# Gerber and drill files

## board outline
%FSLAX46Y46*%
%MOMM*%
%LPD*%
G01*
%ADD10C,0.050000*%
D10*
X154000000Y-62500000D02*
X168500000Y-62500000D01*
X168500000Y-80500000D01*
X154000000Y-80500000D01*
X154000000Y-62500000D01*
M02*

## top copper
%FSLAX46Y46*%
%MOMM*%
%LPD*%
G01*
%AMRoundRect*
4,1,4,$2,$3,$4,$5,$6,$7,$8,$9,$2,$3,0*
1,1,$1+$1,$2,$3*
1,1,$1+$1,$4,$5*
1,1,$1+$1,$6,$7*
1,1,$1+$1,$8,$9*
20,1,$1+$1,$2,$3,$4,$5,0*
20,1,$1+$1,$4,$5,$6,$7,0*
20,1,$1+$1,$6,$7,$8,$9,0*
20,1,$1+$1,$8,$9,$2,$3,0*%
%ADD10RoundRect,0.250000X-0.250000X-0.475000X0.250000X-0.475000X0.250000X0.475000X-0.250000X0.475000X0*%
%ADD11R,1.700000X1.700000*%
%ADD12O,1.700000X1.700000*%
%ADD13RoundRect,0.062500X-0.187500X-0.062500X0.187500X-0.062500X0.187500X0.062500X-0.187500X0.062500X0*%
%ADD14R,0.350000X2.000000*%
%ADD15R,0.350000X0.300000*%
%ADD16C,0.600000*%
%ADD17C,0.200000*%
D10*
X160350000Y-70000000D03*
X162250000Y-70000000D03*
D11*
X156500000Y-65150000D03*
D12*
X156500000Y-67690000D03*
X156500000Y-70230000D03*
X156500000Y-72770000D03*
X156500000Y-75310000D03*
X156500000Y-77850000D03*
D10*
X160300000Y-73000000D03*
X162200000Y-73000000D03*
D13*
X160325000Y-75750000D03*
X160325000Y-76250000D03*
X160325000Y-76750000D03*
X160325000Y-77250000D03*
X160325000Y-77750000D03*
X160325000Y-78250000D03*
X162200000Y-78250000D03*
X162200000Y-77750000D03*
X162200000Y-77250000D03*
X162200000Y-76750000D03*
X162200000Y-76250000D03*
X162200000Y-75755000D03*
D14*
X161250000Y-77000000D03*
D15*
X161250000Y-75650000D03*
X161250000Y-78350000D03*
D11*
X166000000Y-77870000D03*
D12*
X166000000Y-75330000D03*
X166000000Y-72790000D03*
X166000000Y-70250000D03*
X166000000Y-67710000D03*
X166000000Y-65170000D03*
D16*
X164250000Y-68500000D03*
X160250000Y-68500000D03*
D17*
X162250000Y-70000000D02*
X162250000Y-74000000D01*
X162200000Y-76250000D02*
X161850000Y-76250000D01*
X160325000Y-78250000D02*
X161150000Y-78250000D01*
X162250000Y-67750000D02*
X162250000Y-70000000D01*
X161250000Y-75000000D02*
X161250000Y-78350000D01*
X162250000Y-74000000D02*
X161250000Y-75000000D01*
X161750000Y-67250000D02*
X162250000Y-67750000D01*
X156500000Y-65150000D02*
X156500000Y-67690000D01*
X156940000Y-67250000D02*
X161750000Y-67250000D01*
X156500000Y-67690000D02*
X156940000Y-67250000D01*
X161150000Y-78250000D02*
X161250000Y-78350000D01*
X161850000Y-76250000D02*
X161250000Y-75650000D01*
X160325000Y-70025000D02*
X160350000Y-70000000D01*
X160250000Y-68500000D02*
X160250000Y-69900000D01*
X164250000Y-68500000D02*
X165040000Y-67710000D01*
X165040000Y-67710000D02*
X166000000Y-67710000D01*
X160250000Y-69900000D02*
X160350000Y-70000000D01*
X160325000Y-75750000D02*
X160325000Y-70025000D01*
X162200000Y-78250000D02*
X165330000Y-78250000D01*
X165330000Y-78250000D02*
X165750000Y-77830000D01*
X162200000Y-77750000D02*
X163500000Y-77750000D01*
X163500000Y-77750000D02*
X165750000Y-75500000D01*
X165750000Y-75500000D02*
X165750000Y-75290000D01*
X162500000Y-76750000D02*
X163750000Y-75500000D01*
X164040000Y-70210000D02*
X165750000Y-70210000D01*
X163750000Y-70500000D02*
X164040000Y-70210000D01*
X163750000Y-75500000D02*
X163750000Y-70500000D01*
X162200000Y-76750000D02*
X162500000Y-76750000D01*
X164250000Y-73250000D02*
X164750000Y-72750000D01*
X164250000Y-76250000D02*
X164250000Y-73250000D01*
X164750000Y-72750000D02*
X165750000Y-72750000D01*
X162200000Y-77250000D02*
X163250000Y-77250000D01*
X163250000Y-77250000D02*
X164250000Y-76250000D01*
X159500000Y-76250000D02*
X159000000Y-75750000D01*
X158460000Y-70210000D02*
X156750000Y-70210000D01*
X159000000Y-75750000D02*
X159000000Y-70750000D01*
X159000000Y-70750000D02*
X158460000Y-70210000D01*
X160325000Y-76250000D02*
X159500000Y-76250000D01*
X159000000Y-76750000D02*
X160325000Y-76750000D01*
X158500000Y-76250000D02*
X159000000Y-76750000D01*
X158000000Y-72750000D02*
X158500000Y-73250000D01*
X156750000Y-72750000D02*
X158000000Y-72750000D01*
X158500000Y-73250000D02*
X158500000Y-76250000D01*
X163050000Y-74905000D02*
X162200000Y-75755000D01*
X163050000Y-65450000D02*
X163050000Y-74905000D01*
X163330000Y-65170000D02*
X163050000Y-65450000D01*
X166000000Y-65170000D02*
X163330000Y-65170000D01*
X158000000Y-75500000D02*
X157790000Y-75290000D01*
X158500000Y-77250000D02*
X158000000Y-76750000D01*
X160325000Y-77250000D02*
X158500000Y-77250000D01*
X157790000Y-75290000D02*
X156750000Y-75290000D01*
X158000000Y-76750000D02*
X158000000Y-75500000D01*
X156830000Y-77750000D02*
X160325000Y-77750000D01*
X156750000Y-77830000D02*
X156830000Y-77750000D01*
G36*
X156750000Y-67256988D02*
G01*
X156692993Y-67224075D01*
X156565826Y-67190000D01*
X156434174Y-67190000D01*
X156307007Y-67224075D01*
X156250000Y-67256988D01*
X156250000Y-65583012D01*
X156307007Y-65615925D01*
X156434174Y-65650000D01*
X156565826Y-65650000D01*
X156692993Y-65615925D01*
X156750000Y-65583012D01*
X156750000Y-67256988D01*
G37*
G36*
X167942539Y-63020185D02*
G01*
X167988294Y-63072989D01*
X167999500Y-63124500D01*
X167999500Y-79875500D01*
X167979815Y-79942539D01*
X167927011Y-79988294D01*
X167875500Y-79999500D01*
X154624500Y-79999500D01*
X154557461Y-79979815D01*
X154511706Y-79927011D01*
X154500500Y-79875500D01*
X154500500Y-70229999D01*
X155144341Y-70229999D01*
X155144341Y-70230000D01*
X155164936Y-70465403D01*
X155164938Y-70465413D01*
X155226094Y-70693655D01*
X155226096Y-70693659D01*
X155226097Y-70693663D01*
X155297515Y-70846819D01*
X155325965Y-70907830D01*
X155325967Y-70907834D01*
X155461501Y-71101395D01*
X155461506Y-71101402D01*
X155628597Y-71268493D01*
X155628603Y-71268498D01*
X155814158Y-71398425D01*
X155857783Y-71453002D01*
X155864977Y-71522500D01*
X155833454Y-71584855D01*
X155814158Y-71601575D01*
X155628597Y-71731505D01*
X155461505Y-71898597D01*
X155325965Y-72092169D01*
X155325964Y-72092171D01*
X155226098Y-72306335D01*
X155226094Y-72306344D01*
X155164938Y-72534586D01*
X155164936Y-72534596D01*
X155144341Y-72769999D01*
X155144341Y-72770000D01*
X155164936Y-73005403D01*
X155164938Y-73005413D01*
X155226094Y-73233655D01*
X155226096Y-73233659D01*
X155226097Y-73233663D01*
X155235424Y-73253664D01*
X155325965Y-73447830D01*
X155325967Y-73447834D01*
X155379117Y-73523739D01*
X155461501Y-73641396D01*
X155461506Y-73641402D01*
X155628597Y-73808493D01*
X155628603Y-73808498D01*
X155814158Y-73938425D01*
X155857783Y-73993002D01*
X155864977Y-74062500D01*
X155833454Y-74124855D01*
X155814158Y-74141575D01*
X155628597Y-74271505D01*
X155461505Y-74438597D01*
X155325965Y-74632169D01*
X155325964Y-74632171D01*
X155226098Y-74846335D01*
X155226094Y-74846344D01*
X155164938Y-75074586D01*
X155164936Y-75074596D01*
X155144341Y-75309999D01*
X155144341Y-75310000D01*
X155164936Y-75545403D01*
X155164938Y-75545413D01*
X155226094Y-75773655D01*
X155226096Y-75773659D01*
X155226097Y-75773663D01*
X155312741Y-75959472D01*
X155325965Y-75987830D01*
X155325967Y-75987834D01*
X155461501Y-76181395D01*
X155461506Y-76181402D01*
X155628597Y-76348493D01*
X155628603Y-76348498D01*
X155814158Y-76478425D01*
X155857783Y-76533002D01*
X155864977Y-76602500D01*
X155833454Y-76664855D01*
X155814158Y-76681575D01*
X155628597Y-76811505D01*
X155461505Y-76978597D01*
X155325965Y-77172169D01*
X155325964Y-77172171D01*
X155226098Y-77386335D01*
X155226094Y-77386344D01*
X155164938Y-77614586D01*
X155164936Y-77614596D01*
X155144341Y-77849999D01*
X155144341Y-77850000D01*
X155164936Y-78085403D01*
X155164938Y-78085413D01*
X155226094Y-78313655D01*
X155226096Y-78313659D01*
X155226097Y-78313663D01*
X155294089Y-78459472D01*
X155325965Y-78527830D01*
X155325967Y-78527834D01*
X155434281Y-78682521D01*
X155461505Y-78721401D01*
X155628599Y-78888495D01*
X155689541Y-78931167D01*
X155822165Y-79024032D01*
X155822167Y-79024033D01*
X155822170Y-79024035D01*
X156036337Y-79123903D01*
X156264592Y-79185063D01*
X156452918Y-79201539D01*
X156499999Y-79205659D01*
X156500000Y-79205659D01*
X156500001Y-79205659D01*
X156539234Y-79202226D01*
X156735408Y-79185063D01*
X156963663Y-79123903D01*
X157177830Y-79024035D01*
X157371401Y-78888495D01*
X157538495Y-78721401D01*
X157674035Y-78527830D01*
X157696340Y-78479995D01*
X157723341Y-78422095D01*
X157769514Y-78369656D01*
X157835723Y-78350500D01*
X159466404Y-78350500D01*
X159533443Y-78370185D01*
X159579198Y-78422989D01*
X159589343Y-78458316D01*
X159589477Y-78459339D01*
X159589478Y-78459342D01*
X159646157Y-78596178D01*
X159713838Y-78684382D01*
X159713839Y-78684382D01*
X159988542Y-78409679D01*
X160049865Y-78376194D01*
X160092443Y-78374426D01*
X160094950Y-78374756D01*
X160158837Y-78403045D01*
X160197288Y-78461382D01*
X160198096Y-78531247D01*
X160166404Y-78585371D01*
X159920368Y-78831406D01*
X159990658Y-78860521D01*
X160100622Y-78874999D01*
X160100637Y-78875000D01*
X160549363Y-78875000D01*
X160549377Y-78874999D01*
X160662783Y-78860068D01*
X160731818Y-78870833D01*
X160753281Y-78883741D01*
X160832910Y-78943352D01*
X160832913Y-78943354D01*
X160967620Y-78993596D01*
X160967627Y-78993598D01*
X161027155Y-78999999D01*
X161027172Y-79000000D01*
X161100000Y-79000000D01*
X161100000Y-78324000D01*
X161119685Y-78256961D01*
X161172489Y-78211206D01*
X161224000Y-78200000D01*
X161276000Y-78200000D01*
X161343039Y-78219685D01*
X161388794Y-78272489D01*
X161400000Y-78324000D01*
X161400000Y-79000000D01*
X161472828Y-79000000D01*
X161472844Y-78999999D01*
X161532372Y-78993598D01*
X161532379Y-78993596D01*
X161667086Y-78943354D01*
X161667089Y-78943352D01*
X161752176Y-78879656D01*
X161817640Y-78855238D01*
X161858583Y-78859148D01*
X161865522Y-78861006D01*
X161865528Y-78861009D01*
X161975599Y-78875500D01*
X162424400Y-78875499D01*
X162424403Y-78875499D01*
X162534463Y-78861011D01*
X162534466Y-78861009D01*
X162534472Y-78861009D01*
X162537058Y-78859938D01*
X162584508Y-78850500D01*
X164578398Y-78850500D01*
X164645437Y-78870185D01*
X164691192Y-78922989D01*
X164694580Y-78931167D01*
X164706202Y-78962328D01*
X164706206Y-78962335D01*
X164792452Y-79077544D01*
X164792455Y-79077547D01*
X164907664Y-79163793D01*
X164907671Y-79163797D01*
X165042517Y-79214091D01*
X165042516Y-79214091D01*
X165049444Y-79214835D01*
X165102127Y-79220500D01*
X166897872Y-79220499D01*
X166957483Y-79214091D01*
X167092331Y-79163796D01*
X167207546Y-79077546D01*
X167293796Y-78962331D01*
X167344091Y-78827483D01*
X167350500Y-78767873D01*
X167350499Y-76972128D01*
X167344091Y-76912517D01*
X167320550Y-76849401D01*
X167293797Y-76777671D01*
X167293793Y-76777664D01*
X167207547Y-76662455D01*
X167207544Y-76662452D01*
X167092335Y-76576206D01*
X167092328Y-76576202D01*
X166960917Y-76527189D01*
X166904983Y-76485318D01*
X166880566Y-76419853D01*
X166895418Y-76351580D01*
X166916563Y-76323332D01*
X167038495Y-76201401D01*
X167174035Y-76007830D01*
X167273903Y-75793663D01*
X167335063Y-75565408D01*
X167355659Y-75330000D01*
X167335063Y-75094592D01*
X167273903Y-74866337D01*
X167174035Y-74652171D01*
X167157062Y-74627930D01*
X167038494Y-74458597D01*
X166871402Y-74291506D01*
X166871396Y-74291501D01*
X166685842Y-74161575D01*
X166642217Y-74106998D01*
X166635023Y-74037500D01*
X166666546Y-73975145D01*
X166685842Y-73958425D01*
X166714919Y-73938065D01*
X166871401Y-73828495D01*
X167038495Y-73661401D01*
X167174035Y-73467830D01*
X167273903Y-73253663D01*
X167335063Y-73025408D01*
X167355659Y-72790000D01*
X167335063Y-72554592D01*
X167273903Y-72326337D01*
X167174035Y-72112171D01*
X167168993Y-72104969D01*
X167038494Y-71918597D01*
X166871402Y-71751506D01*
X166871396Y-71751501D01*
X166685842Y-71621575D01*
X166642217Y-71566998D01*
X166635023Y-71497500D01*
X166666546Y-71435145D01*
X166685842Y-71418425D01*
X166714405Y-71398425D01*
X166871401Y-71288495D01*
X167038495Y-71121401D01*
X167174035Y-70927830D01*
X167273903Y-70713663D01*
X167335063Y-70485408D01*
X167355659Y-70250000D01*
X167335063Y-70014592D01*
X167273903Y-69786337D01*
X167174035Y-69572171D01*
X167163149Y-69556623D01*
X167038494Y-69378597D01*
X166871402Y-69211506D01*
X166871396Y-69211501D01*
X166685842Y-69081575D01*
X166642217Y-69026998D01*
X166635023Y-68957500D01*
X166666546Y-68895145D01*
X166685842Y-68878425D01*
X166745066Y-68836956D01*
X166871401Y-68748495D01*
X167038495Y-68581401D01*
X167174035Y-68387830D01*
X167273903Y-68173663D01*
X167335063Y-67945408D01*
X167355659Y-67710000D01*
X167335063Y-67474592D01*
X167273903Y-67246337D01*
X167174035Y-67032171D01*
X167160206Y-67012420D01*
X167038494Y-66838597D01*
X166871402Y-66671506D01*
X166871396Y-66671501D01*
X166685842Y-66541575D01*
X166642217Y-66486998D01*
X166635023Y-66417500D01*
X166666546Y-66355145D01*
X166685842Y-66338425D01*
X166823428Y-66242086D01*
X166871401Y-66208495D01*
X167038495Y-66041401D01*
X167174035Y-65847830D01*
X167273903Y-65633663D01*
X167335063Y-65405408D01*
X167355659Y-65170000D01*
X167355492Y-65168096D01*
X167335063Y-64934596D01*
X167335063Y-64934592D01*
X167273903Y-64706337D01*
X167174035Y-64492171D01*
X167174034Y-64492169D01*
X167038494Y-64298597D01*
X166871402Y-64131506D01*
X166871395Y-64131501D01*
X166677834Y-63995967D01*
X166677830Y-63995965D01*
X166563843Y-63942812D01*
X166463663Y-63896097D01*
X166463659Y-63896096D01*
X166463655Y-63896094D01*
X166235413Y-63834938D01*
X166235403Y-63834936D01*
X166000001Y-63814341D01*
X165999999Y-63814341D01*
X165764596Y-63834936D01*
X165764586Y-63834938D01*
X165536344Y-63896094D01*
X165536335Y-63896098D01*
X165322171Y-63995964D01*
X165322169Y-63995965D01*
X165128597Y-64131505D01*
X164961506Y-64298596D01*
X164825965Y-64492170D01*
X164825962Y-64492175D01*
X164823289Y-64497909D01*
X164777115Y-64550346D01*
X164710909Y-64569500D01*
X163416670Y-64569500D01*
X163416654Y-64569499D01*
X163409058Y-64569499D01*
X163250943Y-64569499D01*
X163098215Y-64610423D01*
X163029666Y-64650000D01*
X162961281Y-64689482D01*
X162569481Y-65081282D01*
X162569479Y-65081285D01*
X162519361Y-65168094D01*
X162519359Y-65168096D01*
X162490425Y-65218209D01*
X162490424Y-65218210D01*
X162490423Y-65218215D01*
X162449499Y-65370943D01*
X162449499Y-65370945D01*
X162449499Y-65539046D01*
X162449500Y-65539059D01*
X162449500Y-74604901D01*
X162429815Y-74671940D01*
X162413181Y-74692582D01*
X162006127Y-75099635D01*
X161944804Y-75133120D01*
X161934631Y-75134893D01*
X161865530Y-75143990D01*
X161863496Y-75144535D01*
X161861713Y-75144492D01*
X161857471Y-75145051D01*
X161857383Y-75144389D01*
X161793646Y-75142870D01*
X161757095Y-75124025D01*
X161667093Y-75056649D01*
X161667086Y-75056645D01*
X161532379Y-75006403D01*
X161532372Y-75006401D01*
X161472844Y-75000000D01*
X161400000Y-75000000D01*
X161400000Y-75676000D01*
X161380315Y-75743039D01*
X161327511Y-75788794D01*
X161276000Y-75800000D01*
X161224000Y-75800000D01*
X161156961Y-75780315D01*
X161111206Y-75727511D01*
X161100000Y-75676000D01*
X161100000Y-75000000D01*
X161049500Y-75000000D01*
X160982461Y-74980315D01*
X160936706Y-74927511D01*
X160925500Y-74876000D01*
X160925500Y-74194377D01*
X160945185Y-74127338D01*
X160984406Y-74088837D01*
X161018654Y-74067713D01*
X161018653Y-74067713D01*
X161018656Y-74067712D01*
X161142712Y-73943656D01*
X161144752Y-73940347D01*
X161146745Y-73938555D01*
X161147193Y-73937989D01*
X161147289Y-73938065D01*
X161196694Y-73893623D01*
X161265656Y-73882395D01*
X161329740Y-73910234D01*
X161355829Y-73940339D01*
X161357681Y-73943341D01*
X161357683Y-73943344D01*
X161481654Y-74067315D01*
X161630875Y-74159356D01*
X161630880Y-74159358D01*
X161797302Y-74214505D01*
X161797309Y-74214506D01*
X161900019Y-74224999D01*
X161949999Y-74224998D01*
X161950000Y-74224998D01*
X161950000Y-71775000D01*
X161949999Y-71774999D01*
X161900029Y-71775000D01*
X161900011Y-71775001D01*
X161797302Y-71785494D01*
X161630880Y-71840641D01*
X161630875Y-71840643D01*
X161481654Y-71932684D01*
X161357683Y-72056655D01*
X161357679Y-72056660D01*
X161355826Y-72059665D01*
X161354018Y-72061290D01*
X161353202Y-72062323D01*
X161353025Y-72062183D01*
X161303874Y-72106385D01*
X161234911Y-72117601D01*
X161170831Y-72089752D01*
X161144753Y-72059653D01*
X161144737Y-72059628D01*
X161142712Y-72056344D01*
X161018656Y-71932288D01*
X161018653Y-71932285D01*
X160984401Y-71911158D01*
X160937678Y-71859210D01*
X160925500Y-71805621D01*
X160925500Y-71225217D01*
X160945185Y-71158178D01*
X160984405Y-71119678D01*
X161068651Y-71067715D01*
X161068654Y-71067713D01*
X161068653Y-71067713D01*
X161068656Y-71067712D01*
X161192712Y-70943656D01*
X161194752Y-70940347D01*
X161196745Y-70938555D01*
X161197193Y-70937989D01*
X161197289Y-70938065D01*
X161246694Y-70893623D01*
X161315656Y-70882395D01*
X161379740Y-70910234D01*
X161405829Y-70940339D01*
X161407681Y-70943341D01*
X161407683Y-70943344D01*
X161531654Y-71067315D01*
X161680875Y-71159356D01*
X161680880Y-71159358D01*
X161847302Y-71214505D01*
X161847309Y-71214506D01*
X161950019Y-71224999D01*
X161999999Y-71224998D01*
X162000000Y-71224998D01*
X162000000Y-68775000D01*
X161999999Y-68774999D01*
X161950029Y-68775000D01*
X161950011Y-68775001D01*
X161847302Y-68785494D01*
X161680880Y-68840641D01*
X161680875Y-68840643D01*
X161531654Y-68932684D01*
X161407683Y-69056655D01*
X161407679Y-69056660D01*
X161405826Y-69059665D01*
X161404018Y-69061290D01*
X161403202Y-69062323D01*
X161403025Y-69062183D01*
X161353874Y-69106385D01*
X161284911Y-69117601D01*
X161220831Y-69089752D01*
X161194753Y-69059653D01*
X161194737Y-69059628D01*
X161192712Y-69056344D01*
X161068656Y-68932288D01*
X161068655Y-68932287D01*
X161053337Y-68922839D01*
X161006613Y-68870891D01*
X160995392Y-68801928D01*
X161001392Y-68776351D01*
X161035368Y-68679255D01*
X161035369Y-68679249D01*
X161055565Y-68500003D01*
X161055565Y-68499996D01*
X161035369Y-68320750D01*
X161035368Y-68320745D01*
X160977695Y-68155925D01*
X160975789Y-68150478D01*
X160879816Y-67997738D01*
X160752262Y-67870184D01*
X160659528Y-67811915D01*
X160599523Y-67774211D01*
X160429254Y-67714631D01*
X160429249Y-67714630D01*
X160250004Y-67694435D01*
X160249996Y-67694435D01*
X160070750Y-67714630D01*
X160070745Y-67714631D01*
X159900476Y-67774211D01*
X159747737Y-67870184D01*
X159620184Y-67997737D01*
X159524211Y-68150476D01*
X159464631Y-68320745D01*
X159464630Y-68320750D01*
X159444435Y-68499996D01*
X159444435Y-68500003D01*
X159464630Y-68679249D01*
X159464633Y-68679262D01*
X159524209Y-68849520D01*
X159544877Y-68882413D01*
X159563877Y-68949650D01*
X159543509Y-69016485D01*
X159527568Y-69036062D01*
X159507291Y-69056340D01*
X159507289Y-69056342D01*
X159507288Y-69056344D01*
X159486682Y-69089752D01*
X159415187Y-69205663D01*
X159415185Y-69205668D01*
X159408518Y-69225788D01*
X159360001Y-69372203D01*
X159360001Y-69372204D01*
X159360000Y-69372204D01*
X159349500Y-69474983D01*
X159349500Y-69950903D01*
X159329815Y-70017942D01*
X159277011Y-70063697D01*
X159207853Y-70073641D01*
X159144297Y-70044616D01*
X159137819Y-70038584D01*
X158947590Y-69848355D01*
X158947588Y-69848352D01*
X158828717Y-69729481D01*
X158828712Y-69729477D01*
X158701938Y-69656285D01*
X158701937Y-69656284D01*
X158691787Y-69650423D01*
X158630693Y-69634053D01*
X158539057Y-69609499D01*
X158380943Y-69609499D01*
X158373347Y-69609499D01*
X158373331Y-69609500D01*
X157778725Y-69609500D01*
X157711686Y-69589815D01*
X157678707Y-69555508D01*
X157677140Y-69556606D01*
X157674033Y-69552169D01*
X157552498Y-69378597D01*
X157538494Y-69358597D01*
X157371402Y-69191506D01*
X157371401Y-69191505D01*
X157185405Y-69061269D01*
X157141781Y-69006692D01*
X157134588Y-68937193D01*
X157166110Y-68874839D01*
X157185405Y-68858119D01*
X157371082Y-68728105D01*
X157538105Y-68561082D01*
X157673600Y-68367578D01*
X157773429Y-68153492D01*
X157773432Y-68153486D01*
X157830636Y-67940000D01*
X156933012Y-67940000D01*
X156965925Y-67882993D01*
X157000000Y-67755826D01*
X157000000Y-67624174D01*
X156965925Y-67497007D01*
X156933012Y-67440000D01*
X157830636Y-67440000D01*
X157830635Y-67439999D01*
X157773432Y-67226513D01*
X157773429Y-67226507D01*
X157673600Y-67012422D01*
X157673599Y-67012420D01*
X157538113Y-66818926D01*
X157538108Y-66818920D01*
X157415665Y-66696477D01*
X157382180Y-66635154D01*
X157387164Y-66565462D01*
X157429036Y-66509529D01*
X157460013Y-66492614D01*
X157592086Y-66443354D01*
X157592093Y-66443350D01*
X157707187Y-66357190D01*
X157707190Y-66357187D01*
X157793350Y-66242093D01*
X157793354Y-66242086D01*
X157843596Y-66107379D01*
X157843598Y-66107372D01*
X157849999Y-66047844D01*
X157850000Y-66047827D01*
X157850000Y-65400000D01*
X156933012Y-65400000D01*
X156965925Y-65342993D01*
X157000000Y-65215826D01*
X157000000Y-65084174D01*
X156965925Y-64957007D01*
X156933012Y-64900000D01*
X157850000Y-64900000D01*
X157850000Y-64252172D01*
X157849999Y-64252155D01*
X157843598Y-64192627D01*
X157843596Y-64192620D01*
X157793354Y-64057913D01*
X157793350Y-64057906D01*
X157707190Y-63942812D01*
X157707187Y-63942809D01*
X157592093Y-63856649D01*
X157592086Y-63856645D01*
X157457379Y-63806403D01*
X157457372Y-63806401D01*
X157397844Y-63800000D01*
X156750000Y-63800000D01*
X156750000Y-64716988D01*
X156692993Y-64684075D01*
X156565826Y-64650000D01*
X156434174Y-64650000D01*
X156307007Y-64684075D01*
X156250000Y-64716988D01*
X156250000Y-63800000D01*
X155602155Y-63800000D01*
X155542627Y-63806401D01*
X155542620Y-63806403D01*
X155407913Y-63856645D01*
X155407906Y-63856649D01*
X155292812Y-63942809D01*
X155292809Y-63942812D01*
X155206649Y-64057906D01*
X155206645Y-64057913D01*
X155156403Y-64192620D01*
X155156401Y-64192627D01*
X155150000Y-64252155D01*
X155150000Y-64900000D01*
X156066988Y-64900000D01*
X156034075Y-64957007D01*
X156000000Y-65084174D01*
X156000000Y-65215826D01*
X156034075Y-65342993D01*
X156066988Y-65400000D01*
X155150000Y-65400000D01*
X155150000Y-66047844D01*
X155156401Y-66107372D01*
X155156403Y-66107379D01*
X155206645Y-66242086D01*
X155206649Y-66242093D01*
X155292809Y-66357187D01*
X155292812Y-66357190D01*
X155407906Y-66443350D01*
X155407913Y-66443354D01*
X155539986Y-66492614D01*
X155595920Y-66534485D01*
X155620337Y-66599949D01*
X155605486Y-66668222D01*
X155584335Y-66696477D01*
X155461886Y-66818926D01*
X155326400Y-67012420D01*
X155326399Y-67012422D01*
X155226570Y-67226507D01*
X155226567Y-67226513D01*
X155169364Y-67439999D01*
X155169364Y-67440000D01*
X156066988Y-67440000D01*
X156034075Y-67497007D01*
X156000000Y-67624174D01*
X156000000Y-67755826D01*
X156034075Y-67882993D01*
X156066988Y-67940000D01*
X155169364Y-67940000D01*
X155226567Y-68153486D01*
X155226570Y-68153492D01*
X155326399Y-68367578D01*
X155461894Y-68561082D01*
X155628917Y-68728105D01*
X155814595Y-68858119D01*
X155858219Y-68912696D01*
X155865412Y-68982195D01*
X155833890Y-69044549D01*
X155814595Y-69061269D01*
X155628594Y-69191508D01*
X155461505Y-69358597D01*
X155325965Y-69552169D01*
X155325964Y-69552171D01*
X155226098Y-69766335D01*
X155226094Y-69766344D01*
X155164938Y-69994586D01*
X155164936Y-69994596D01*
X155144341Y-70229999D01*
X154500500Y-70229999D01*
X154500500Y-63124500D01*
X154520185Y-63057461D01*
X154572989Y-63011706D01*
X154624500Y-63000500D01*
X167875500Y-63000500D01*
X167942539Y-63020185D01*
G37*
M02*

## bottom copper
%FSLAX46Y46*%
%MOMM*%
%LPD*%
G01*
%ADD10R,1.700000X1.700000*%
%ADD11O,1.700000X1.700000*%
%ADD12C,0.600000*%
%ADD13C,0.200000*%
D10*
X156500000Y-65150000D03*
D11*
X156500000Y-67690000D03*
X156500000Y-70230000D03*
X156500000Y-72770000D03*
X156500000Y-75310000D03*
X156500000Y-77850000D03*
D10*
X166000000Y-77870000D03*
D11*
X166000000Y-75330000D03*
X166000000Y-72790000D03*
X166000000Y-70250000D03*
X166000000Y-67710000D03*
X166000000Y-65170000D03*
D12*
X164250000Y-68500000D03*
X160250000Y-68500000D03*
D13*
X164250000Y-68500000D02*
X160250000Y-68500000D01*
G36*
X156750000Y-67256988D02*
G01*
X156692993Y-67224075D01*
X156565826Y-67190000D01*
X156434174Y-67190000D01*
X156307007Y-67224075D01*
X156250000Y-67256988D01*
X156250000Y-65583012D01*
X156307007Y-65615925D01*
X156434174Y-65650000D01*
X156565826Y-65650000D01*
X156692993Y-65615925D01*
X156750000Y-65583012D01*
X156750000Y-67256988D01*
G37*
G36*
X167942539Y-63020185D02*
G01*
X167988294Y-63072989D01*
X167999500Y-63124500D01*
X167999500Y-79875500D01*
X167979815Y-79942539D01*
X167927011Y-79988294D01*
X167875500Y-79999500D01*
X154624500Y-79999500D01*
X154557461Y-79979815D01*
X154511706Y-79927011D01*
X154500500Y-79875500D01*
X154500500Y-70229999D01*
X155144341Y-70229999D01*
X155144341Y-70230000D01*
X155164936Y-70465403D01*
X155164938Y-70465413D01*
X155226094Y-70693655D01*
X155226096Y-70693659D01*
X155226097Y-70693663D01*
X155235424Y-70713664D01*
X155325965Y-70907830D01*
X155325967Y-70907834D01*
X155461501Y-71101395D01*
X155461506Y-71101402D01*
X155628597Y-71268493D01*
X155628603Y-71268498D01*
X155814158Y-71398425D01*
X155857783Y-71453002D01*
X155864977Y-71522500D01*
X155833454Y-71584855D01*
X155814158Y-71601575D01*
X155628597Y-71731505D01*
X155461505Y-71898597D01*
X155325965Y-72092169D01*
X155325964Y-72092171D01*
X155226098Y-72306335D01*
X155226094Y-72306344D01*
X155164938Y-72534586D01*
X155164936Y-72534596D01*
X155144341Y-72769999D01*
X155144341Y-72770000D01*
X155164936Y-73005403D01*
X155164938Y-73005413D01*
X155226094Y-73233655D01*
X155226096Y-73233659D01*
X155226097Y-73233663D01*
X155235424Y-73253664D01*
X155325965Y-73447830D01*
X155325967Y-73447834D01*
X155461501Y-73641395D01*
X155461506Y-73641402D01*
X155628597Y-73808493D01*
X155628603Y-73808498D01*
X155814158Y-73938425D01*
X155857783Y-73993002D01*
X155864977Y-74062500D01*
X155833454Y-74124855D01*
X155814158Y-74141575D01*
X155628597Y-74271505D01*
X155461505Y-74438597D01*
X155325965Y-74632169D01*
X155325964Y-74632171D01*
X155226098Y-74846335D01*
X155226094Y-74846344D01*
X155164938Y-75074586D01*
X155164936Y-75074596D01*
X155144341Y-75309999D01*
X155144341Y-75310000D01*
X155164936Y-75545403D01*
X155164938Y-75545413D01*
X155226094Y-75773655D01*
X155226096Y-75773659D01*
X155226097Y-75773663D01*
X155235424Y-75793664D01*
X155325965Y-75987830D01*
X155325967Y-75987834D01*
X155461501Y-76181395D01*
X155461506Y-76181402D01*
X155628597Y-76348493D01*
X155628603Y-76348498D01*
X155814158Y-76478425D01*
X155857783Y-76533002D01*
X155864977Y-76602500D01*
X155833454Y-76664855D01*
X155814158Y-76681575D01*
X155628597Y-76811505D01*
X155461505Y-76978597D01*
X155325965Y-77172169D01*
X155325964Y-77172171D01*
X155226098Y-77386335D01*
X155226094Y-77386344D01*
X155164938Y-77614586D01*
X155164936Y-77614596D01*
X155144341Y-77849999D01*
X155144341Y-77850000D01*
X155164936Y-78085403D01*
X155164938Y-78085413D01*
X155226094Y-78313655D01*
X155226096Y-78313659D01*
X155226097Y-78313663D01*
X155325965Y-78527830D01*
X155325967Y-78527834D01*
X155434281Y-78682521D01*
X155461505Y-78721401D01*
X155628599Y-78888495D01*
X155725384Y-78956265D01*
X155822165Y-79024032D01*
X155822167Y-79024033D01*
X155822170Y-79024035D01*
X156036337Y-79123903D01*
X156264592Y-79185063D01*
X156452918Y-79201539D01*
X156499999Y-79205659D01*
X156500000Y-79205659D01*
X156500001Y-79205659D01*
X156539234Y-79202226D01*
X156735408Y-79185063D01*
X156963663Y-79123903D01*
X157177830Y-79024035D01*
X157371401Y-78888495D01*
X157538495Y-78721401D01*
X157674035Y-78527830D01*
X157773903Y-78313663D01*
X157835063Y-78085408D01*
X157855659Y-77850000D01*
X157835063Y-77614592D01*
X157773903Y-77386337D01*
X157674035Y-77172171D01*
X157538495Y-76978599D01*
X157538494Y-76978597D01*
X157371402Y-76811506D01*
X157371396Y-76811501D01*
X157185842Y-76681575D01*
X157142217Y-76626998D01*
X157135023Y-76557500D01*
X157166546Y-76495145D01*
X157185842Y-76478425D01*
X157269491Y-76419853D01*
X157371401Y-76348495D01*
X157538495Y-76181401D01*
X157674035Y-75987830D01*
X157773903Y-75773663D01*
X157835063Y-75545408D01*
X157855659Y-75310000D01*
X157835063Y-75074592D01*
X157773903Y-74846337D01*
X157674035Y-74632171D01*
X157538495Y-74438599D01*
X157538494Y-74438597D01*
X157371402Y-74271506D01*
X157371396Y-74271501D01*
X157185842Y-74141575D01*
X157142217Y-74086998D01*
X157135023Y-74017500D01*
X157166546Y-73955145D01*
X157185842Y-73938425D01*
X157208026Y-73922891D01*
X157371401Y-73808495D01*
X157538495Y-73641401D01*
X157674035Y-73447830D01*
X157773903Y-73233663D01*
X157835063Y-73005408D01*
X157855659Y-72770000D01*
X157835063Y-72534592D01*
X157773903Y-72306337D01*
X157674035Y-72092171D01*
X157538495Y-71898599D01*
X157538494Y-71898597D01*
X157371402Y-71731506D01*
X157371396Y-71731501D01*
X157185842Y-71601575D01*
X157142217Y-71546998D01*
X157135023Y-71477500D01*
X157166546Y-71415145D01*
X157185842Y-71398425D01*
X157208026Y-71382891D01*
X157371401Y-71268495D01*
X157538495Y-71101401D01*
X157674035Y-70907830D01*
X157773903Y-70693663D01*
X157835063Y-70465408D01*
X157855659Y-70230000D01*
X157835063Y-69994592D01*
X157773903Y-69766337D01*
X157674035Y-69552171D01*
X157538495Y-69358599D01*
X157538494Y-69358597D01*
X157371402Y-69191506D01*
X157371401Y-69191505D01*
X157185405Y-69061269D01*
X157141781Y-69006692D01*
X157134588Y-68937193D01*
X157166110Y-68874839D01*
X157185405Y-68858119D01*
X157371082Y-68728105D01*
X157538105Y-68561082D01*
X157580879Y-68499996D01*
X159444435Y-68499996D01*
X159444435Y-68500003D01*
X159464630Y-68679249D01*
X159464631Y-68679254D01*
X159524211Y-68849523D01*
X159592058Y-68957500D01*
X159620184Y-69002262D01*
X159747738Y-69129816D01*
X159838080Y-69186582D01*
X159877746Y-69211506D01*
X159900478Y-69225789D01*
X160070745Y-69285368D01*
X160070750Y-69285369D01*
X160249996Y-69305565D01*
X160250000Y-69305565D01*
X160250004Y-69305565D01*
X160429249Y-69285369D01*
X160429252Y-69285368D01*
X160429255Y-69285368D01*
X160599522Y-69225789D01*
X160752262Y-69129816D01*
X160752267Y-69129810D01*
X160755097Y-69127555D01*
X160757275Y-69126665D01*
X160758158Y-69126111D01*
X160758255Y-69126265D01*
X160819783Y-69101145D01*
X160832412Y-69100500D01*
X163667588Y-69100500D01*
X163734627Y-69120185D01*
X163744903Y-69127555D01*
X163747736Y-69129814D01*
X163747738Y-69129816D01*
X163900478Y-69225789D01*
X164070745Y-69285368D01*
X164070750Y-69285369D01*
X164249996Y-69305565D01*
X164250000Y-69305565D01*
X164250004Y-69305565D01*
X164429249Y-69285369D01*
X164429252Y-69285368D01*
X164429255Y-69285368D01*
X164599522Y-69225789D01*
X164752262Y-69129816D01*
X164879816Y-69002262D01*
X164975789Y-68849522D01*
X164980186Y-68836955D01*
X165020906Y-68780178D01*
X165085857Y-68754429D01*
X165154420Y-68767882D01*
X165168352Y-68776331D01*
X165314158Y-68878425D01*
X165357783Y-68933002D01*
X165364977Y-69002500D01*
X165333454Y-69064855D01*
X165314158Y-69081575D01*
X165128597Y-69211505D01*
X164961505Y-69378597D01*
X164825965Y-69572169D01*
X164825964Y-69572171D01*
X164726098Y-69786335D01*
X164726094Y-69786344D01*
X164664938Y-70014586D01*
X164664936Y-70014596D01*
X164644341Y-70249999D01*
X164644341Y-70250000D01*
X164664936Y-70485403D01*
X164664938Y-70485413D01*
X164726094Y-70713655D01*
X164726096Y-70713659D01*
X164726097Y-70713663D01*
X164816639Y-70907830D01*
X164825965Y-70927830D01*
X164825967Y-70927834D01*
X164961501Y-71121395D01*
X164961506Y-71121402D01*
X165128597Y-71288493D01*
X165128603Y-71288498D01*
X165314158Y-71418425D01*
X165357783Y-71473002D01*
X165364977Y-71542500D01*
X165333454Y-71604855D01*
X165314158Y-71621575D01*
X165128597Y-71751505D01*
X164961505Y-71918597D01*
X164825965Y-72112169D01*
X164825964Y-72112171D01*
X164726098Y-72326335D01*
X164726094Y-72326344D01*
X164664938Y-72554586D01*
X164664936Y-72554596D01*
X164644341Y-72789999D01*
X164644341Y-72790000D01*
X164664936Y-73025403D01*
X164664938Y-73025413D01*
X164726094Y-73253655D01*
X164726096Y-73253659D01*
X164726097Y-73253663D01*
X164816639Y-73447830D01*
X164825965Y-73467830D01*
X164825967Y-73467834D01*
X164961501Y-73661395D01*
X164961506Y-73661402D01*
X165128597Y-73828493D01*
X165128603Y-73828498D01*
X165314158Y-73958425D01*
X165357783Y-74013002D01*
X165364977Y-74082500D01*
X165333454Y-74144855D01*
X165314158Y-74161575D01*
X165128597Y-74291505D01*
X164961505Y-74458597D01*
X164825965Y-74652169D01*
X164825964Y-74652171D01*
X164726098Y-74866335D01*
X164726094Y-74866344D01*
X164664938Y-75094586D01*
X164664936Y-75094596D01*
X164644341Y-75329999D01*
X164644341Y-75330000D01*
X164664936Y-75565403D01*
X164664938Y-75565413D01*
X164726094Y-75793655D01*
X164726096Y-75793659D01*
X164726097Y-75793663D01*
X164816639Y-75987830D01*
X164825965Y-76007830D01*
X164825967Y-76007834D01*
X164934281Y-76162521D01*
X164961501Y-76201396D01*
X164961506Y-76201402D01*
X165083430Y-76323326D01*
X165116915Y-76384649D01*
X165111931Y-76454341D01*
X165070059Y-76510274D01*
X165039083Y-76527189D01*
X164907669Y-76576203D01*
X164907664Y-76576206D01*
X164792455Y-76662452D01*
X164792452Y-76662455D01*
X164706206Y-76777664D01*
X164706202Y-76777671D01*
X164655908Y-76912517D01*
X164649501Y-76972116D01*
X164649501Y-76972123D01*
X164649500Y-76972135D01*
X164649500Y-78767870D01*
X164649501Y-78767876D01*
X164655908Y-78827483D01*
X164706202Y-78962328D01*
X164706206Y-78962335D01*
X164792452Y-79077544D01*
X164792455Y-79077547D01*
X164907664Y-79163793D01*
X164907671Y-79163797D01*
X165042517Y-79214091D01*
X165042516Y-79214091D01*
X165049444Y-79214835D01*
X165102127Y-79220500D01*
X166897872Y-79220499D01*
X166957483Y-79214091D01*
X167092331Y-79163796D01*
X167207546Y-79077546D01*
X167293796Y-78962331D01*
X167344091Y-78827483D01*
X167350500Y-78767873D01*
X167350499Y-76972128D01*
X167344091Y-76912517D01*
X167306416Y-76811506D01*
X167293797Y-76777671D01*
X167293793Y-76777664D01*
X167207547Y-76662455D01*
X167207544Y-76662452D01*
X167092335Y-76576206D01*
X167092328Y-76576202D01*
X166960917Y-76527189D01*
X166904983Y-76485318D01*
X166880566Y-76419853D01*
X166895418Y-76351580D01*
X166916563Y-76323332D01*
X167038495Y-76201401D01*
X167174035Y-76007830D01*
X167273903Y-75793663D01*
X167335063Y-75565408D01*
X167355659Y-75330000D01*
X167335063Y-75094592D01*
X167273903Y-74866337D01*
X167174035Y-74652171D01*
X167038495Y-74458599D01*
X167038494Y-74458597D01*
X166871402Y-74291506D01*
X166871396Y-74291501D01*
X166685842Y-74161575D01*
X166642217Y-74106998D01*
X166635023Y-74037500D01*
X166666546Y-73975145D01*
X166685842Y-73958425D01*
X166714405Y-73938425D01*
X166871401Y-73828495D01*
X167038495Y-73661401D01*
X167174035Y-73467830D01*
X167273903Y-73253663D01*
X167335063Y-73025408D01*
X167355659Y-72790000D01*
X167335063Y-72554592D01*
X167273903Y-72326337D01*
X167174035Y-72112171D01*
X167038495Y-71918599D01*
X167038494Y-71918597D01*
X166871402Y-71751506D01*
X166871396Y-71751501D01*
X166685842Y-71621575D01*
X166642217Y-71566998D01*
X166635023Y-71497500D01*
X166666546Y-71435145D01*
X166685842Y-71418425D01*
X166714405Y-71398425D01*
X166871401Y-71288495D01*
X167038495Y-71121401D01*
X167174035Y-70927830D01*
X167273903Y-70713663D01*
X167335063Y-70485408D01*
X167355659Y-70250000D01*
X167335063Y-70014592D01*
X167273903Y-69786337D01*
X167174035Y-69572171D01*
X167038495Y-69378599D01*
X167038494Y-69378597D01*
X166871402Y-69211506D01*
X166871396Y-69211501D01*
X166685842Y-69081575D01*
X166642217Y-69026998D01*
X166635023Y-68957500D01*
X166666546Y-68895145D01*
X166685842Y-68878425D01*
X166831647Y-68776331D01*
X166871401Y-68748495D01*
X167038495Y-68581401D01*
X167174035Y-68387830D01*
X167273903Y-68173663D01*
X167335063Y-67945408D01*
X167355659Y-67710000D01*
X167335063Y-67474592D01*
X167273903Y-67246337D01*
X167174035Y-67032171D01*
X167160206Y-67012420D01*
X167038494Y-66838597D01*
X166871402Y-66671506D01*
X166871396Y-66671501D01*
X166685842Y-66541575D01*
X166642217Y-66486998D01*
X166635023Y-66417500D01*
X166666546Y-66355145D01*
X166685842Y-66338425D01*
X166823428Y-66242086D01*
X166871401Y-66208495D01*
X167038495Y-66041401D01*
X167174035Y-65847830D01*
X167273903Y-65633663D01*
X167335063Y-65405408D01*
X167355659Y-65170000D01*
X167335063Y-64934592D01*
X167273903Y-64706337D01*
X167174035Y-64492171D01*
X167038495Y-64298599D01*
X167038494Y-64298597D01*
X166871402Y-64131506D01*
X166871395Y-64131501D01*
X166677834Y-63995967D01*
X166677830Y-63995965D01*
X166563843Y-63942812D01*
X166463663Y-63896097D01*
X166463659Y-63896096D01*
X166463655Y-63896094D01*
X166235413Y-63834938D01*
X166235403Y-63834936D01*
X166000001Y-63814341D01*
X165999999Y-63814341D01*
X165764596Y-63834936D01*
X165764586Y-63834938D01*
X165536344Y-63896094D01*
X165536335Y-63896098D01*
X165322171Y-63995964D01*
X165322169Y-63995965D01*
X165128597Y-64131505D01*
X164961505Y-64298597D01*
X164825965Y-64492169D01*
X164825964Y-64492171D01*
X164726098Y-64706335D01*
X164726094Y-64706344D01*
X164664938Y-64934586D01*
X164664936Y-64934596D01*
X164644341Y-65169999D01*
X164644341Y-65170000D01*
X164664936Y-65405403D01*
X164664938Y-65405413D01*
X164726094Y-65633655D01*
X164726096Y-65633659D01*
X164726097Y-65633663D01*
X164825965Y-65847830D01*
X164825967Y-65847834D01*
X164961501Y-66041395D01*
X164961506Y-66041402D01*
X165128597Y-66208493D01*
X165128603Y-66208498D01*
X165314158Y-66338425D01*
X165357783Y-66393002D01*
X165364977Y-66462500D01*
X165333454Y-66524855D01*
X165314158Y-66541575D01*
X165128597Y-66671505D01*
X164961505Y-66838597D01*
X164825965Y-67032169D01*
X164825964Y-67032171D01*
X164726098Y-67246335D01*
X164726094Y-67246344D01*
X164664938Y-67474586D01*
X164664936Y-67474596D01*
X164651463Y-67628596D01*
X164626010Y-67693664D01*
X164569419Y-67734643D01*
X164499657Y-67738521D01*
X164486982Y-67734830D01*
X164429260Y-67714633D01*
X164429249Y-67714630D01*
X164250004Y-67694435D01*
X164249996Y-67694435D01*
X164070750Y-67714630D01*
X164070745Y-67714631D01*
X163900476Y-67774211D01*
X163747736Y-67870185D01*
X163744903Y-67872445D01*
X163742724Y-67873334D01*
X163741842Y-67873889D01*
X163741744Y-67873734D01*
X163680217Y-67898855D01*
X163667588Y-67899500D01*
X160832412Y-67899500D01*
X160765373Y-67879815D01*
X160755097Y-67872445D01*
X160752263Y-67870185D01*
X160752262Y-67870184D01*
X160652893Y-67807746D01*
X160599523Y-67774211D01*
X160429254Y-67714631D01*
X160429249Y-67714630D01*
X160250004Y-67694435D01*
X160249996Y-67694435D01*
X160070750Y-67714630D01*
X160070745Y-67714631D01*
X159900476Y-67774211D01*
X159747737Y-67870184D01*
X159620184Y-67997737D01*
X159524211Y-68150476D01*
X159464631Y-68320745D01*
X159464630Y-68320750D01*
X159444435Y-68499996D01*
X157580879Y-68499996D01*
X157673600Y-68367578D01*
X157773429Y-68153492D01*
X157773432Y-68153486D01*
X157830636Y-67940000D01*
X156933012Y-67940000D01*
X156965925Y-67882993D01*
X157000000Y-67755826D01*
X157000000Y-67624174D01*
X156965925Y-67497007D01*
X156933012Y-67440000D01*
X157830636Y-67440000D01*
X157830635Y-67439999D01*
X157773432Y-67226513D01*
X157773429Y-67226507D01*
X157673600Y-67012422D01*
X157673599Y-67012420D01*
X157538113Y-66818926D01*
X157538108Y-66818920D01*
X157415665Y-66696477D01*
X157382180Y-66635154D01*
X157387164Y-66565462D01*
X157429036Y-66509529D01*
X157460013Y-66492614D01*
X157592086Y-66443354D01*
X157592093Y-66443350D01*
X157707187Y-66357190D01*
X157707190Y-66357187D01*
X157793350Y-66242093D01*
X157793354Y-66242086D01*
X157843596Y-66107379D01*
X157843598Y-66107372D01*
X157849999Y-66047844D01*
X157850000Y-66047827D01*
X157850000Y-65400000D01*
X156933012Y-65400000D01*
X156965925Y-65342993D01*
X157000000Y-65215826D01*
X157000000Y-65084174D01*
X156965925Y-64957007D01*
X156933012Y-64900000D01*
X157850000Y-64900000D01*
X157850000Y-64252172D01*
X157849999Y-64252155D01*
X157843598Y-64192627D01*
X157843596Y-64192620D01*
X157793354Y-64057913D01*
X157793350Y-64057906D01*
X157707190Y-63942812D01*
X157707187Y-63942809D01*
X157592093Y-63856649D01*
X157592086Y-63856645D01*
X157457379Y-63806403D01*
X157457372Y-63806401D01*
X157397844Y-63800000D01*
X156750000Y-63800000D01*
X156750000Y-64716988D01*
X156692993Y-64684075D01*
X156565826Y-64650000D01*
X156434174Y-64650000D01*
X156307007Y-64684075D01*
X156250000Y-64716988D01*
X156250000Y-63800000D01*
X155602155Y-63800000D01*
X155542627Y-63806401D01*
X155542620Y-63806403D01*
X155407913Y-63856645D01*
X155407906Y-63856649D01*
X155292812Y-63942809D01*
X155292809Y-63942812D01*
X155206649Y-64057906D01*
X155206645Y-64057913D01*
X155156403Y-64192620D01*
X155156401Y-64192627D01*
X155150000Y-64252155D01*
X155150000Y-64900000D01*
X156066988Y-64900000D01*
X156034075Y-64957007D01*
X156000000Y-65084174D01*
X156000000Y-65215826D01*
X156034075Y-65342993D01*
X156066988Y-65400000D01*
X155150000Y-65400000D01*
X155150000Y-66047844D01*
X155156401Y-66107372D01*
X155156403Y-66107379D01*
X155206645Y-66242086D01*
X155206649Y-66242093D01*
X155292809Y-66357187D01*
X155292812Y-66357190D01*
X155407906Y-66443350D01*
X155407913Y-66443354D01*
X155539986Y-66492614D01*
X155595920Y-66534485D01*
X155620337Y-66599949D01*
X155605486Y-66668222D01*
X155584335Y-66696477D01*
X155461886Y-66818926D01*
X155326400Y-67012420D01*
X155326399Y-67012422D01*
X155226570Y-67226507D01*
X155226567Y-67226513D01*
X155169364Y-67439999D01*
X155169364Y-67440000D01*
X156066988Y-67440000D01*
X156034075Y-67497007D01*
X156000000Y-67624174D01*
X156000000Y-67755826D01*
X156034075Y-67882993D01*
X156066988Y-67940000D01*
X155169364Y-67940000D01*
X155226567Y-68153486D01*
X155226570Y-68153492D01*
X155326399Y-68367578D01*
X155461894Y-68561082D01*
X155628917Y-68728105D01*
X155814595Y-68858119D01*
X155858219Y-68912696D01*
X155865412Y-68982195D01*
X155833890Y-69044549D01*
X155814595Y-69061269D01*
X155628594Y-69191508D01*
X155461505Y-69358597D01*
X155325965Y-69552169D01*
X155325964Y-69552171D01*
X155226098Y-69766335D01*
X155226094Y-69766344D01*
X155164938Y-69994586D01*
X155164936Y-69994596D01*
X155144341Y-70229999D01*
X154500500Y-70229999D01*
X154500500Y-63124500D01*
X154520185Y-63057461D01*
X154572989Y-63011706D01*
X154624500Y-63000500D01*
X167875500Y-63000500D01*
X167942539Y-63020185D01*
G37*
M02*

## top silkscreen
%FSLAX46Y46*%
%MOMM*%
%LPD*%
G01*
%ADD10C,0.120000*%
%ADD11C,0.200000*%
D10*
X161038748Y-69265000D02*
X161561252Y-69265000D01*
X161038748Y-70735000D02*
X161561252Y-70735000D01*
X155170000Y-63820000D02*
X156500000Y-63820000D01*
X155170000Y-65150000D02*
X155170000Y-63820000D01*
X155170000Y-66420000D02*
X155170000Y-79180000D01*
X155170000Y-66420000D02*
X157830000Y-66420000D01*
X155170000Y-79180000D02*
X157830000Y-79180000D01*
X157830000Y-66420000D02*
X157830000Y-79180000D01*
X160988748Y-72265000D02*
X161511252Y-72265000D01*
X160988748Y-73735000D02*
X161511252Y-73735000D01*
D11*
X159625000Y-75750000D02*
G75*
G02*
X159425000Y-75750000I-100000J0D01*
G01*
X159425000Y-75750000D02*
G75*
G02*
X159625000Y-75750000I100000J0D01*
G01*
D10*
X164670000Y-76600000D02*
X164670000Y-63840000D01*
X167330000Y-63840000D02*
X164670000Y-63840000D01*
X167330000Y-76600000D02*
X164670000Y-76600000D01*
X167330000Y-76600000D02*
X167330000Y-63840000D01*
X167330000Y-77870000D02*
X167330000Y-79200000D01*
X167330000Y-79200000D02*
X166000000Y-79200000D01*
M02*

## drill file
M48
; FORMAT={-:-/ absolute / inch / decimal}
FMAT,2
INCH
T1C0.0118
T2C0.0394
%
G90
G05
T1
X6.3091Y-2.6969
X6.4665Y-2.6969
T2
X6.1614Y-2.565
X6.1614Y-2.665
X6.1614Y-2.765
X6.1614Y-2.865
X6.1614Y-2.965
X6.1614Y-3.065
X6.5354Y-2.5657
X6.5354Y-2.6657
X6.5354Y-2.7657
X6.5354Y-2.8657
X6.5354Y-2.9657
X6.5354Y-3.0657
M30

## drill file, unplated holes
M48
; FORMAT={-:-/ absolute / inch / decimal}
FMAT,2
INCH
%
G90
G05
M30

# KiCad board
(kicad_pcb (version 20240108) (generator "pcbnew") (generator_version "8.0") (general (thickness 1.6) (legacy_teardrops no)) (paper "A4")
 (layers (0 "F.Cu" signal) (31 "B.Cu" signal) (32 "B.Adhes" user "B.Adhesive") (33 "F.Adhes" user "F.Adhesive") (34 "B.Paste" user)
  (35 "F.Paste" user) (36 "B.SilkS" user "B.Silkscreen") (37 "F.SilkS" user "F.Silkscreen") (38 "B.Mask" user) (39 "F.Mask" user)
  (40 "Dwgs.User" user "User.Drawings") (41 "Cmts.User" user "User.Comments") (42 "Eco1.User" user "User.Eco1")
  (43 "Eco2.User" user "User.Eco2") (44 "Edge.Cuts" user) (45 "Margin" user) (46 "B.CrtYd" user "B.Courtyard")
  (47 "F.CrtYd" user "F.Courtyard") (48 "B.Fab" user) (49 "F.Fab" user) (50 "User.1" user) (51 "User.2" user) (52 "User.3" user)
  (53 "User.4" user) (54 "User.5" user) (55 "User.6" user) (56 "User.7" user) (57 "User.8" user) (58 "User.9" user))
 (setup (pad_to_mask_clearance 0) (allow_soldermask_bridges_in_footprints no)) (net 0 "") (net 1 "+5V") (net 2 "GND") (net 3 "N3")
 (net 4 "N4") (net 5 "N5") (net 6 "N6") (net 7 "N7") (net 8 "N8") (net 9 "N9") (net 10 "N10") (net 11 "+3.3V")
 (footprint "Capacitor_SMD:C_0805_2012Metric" (layer "F.Cu") (at 161.3 70)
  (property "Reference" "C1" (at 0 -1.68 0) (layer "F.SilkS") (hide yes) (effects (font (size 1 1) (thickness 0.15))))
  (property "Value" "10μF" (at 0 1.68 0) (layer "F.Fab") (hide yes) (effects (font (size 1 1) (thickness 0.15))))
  (fp_line (start -0.261252 -0.735) (end 0.261252 -0.735) (stroke (width 0.12) (type solid)) (layer "F.SilkS"))
  (fp_line (start -0.261252 0.735) (end 0.261252 0.735) (stroke (width 0.12) (type solid)) (layer "F.SilkS"))
  (pad "1" smd roundrect (at -0.95 0) (size 1 1.45) (layers "F.Cu" "F.Paste" "F.Mask") (roundrect_rratio 0.25) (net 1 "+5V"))
  (pad "2" smd roundrect (at 0.95 0) (size 1 1.45) (layers "F.Cu" "F.Paste" "F.Mask") (roundrect_rratio 0.25) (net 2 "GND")))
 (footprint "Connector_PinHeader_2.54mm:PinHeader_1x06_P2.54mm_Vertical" (layer "F.Cu") (at 156.5 65.15)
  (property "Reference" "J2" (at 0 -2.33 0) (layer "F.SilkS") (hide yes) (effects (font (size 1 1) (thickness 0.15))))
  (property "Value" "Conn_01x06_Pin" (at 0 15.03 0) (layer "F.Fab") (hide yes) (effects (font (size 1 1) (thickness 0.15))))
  (fp_line (start -1.33 -1.33) (end 0 -1.33) (stroke (width 0.12) (type solid)) (layer "F.SilkS"))
  (fp_line (start -1.33 0) (end -1.33 -1.33) (stroke (width 0.12) (type solid)) (layer "F.SilkS"))
  (fp_line (start -1.33 1.27) (end -1.33 14.03) (stroke (width 0.12) (type solid)) (layer "F.SilkS"))
  (fp_line (start -1.33 1.27) (end 1.33 1.27) (stroke (width 0.12) (type solid)) (layer "F.SilkS"))
  (fp_line (start -1.33 14.03) (end 1.33 14.03) (stroke (width 0.12) (type solid)) (layer "F.SilkS"))
  (fp_line (start 1.33 1.27) (end 1.33 14.03) (stroke (width 0.12) (type solid)) (layer "F.SilkS"))
  (pad "1" thru_hole rect (at 0 0) (size 1.7 1.7) (drill 1) (layers "*.Cu" "*.Mask") (remove_unused_layers no) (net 2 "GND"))
  (pad "2" thru_hole oval (at 0 2.54) (size 1.7 1.7) (drill 1) (layers "*.Cu" "*.Mask") (remove_unused_layers no) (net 2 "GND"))
  (pad "3" thru_hole oval (at 0 5.08) (size 1.7 1.7) (drill 1) (layers "*.Cu" "*.Mask") (remove_unused_layers no) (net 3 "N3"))
  (pad "4" thru_hole oval (at 0 7.62) (size 1.7 1.7) (drill 1) (layers "*.Cu" "*.Mask") (remove_unused_layers no) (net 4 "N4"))
  (pad "5" thru_hole oval (at 0 10.16) (size 1.7 1.7) (drill 1) (layers "*.Cu" "*.Mask") (remove_unused_layers no) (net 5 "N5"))
  (pad "6" thru_hole oval (at 0 12.7) (size 1.7 1.7) (drill 1) (layers "*.Cu" "*.Mask") (remove_unused_layers no) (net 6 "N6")))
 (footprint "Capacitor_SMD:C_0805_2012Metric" (layer "F.Cu") (at 161.25 73)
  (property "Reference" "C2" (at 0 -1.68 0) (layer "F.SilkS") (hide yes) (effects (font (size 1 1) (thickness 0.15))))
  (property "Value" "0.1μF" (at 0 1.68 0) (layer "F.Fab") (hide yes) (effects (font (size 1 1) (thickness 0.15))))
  (fp_line (start -0.261252 -0.735) (end 0.261252 -0.735) (stroke (width 0.12) (type solid)) (layer "F.SilkS"))
  (fp_line (start -0.261252 0.735) (end 0.261252 0.735) (stroke (width 0.12) (type solid)) (layer "F.SilkS"))
  (pad "1" smd roundrect (at -0.95 0) (size 1 1.45) (layers "F.Cu" "F.Paste" "F.Mask") (roundrect_rratio 0.25) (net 1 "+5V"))
  (pad "2" smd roundrect (at 0.95 0) (size 1 1.45) (layers "F.Cu" "F.Paste" "F.Mask") (roundrect_rratio 0.25) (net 2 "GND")))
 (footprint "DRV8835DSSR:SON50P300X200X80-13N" (layer "F.Cu") (at 161.25 77)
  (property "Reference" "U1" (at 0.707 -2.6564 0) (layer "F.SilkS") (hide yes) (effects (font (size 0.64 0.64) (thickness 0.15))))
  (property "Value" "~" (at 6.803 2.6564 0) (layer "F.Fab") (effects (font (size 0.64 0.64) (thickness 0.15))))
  (fp_circle (center -1.725 -1.25) (end -1.625 -1.25) (stroke (width 0.2) (type solid)) (fill none) (layer "F.SilkS"))
  (pad "1" smd roundrect (at -0.925 -1.25) (size 0.5 0.25) (layers "F.Cu" "F.Paste" "F.Mask") (roundrect_rratio 0.25) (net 1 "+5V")
   (thermal_bridge_angle 45))
  (pad "2" smd roundrect (at -0.925 -0.75) (size 0.5 0.25) (layers "F.Cu" "F.Paste" "F.Mask") (roundrect_rratio 0.25) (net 3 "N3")
   (thermal_bridge_angle 45))
  (pad "3" smd roundrect (at -0.925 -0.25) (size 0.5 0.25) (layers "F.Cu" "F.Paste" "F.Mask") (roundrect_rratio 0.25) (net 4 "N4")
   (thermal_bridge_angle 45))
  (pad "4" smd roundrect (at -0.925 0.25) (size 0.5 0.25) (layers "F.Cu" "F.Paste" "F.Mask") (roundrect_rratio 0.25) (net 5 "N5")
   (thermal_bridge_angle 45))
  (pad "5" smd roundrect (at -0.925 0.75) (size 0.5 0.25) (layers "F.Cu" "F.Paste" "F.Mask") (roundrect_rratio 0.25) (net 6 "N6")
   (thermal_bridge_angle 45))
  (pad "6" smd roundrect (at -0.925 1.25) (size 0.5 0.25) (layers "F.Cu" "F.Paste" "F.Mask") (roundrect_rratio 0.25) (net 2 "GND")
   (thermal_bridge_angle 45))
  (pad "7" smd roundrect (at 0.95 1.25) (size 0.5 0.25) (layers "F.Cu" "F.Paste" "F.Mask") (roundrect_rratio 0.25) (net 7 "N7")
   (thermal_bridge_angle 45))
  (pad "8" smd roundrect (at 0.95 0.75) (size 0.5 0.25) (layers "F.Cu" "F.Paste" "F.Mask") (roundrect_rratio 0.25) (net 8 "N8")
   (thermal_bridge_angle 45))
  (pad "9" smd roundrect (at 0.95 0.25) (size 0.5 0.25) (layers "F.Cu" "F.Paste" "F.Mask") (roundrect_rratio 0.25) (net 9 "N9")
   (thermal_bridge_angle 45))
  (pad "10" smd roundrect (at 0.95 -0.25) (size 0.5 0.25) (layers "F.Cu" "F.Paste" "F.Mask") (roundrect_rratio 0.25) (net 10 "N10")
   (thermal_bridge_angle 45))
  (pad "11" smd roundrect (at 0.95 -0.75) (size 0.5 0.25) (layers "F.Cu" "F.Paste" "F.Mask") (roundrect_rratio 0.25) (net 2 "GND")
   (thermal_bridge_angle 45))
  (pad "12" smd roundrect (at 0.95 -1.245) (size 0.5 0.25) (layers "F.Cu" "F.Paste" "F.Mask") (roundrect_rratio 0.25) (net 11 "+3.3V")
   (thermal_bridge_angle 45))
  (pad "13" smd rect (at 0 0) (size 0.35 2) (layers "F.Cu") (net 2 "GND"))
  (pad "14" smd rect (at 0 -1.35) (size 0.35 0.3) (layers "F.Cu") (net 2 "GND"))
  (pad "15" smd rect (at 0 1.35) (size 0.35 0.3) (layers "F.Cu") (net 2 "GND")))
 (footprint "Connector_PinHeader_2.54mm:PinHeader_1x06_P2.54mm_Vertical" (layer "F.Cu") (at 166 77.87 180)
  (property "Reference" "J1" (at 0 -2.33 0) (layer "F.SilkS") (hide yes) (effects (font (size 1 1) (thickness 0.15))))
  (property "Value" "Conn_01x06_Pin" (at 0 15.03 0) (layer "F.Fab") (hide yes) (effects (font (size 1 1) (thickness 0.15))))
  (fp_line (start 1.33 1.27) (end 1.33 14.03) (stroke (width 0.12) (type solid)) (layer "F.SilkS"))
  (fp_line (start -1.33 14.03) (end 1.33 14.03) (stroke (width 0.12) (type solid)) (layer "F.SilkS"))
  (fp_line (start -1.33 1.27) (end 1.33 1.27) (stroke (width 0.12) (type solid)) (layer "F.SilkS"))
  (fp_line (start -1.33 1.27) (end -1.33 14.03) (stroke (width 0.12) (type solid)) (layer "F.SilkS"))
  (fp_line (start -1.33 0) (end -1.33 -1.33) (stroke (width 0.12) (type solid)) (layer "F.SilkS"))
  (fp_line (start -1.33 -1.33) (end 0 -1.33) (stroke (width 0.12) (type solid)) (layer "F.SilkS"))
  (pad "1" thru_hole rect (at 0 0 180) (size 1.7 1.7) (drill 1) (layers "*.Cu" "*.Mask") (remove_unused_layers no) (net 7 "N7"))
  (pad "2" thru_hole oval (at 0 2.54 180) (size 1.7 1.7) (drill 1) (layers "*.Cu" "*.Mask") (remove_unused_layers no) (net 8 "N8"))
  (pad "3" thru_hole oval (at 0 5.08 180) (size 1.7 1.7) (drill 1) (layers "*.Cu" "*.Mask") (remove_unused_layers no) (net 9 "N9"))
  (pad "4" thru_hole oval (at 0 7.62 180) (size 1.7 1.7) (drill 1) (layers "*.Cu" "*.Mask") (remove_unused_layers no) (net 10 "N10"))
  (pad "5" thru_hole oval (at 0 10.16 180) (size 1.7 1.7) (drill 1) (layers "*.Cu" "*.Mask") (remove_unused_layers no) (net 1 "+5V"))
  (pad "6" thru_hole oval (at 0 12.7 180) (size 1.7 1.7) (drill 1) (layers "*.Cu" "*.Mask") (remove_unused_layers no) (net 11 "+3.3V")))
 (gr_rect (start 154 62.5) (end 168.5 80.5) (stroke (width 0.05) (type default)) (fill none) (layer "Edge.Cuts"))
 (segment (start 162.25 70) (end 162.25 74) (width 0.2) (layer "F.Cu") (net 2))
 (segment (start 162.2 76.25) (end 161.85 76.25) (width 0.2) (layer "F.Cu") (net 2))
 (segment (start 160.325 78.25) (end 161.15 78.25) (width 0.2) (layer "F.Cu") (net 2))
 (segment (start 162.25 67.75) (end 162.25 70) (width 0.2) (layer "F.Cu") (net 2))
 (segment (start 161.25 75) (end 161.25 78.35) (width 0.2) (layer "F.Cu") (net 2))
 (segment (start 162.25 74) (end 161.25 75) (width 0.2) (layer "F.Cu") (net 2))
 (segment (start 161.75 67.25) (end 162.25 67.75) (width 0.2) (layer "F.Cu") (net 2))
 (segment (start 156.5 65.15) (end 156.5 67.69) (width 0.2) (layer "F.Cu") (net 2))
 (segment (start 156.94 67.25) (end 161.75 67.25) (width 0.2) (layer "F.Cu") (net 2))
 (segment (start 156.5 67.69) (end 156.94 67.25) (width 0.2) (layer "F.Cu") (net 2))
 (segment (start 161.15 78.25) (end 161.25 78.35) (width 0.2) (layer "F.Cu") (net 2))
 (segment (start 161.85 76.25) (end 161.25 75.65) (width 0.2) (layer "F.Cu") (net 2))
 (segment (start 160.325 70.025) (end 160.35 70) (width 0.2) (layer "F.Cu") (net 1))
 (segment (start 160.25 68.5) (end 160.25 69.9) (width 0.2) (layer "F.Cu") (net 1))
 (segment (start 164.25 68.5) (end 165.04 67.71) (width 0.2) (layer "F.Cu") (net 1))
 (segment (start 165.04 67.71) (end 166 67.71) (width 0.2) (layer "F.Cu") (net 1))
 (segment (start 160.25 69.9) (end 160.35 70) (width 0.2) (layer "F.Cu") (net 1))
 (segment (start 160.325 75.75) (end 160.325 70.025) (width 0.2) (layer "F.Cu") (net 1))
 (via (at 164.25 68.5) (size 0.6) (drill 0.3) (layers "F.Cu" "B.Cu") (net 1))
 (via (at 160.25 68.5) (size 0.6) (drill 0.3) (layers "F.Cu" "B.Cu") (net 1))
 (segment (start 164.25 68.5) (end 160.25 68.5) (width 0.2) (layer "B.Cu") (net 1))
 (segment (start 162.2 78.25) (end 165.33 78.25) (width 0.2) (layer "F.Cu") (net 7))
 (segment (start 165.33 78.25) (end 165.75 77.83) (width 0.2) (layer "F.Cu") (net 7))
 (segment (start 162.2 77.75) (end 163.5 77.75) (width 0.2) (layer "F.Cu") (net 8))
 (segment (start 163.5 77.75) (end 165.75 75.5) (width 0.2) (layer "F.Cu") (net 8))
 (segment (start 165.75 75.5) (end 165.75 75.29) (width 0.2) (layer "F.Cu") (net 8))
 (segment (start 162.5 76.75) (end 163.75 75.5) (width 0.2) (layer "F.Cu") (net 10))
 (segment (start 164.04 70.21) (end 165.75 70.21) (width 0.2) (layer "F.Cu") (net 10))
 (segment (start 163.75 70.5) (end 164.04 70.21) (width 0.2) (layer "F.Cu") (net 10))
 (segment (start 163.75 75.5) (end 163.75 70.5) (width 0.2) (layer "F.Cu") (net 10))
 (segment (start 162.2 76.75) (end 162.5 76.75) (width 0.2) (layer "F.Cu") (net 10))
 (segment (start 164.25 73.25) (end 164.75 72.75) (width 0.2) (layer "F.Cu") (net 9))
 (segment (start 164.25 76.25) (end 164.25 73.25) (width 0.2) (layer "F.Cu") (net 9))
 (segment (start 164.75 72.75) (end 165.75 72.75) (width 0.2) (layer "F.Cu") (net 9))
 (segment (start 162.2 77.25) (end 163.25 77.25) (width 0.2) (layer "F.Cu") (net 9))
 (segment (start 163.25 77.25) (end 164.25 76.25) (width 0.2) (layer "F.Cu") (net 9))
 (segment (start 159.5 76.25) (end 159 75.75) (width 0.2) (layer "F.Cu") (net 3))
 (segment (start 158.46 70.21) (end 156.75 70.21) (width 0.2) (layer "F.Cu") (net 3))
 (segment (start 159 75.75) (end 159 70.75) (width 0.2) (layer "F.Cu") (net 3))
 (segment (start 159 70.75) (end 158.46 70.21) (width 0.2) (layer "F.Cu") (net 3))
 (segment (start 160.325 76.25) (end 159.5 76.25) (width 0.2) (layer "F.Cu") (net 3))
 (segment (start 159 76.75) (end 160.325 76.75) (width 0.2) (layer "F.Cu") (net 4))
 (segment (start 158.5 76.25) (end 159 76.75) (width 0.2) (layer "F.Cu") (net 4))
 (segment (start 158 72.75) (end 158.5 73.25) (width 0.2) (layer "F.Cu") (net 4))
 (segment (start 156.75 72.75) (end 158 72.75) (width 0.2) (layer "F.Cu") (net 4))
 (segment (start 158.5 73.25) (end 158.5 76.25) (width 0.2) (layer "F.Cu") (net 4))
 (segment (start 163.05 74.905) (end 162.2 75.755) (width 0.2) (layer "F.Cu") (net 11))
 (segment (start 163.05 65.45) (end 163.05 74.905) (width 0.2) (layer "F.Cu") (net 11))
 (segment (start 163.33 65.17) (end 163.05 65.45) (width 0.2) (layer "F.Cu") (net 11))
 (segment (start 166 65.17) (end 163.33 65.17) (width 0.2) (layer "F.Cu") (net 11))
 (segment (start 158 75.5) (end 157.79 75.29) (width 0.2) (layer "F.Cu") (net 5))
 (segment (start 158.5 77.25) (end 158 76.75) (width 0.2) (layer "F.Cu") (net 5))
 (segment (start 160.325 77.25) (end 158.5 77.25) (width 0.2) (layer "F.Cu") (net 5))
 (segment (start 157.79 75.29) (end 156.75 75.29) (width 0.2) (layer "F.Cu") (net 5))
 (segment (start 158 76.75) (end 158 75.5) (width 0.2) (layer "F.Cu") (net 5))
 (segment (start 156.83 77.75) (end 160.325 77.75) (width 0.2) (layer "F.Cu") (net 6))
 (segment (start 156.75 77.83) (end 156.83 77.75) (width 0.2) (layer "F.Cu") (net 6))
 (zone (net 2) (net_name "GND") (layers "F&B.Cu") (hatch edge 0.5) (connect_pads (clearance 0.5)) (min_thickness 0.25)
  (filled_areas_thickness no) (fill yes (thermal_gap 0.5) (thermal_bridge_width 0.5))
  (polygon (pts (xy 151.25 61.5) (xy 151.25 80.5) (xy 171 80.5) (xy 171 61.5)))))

